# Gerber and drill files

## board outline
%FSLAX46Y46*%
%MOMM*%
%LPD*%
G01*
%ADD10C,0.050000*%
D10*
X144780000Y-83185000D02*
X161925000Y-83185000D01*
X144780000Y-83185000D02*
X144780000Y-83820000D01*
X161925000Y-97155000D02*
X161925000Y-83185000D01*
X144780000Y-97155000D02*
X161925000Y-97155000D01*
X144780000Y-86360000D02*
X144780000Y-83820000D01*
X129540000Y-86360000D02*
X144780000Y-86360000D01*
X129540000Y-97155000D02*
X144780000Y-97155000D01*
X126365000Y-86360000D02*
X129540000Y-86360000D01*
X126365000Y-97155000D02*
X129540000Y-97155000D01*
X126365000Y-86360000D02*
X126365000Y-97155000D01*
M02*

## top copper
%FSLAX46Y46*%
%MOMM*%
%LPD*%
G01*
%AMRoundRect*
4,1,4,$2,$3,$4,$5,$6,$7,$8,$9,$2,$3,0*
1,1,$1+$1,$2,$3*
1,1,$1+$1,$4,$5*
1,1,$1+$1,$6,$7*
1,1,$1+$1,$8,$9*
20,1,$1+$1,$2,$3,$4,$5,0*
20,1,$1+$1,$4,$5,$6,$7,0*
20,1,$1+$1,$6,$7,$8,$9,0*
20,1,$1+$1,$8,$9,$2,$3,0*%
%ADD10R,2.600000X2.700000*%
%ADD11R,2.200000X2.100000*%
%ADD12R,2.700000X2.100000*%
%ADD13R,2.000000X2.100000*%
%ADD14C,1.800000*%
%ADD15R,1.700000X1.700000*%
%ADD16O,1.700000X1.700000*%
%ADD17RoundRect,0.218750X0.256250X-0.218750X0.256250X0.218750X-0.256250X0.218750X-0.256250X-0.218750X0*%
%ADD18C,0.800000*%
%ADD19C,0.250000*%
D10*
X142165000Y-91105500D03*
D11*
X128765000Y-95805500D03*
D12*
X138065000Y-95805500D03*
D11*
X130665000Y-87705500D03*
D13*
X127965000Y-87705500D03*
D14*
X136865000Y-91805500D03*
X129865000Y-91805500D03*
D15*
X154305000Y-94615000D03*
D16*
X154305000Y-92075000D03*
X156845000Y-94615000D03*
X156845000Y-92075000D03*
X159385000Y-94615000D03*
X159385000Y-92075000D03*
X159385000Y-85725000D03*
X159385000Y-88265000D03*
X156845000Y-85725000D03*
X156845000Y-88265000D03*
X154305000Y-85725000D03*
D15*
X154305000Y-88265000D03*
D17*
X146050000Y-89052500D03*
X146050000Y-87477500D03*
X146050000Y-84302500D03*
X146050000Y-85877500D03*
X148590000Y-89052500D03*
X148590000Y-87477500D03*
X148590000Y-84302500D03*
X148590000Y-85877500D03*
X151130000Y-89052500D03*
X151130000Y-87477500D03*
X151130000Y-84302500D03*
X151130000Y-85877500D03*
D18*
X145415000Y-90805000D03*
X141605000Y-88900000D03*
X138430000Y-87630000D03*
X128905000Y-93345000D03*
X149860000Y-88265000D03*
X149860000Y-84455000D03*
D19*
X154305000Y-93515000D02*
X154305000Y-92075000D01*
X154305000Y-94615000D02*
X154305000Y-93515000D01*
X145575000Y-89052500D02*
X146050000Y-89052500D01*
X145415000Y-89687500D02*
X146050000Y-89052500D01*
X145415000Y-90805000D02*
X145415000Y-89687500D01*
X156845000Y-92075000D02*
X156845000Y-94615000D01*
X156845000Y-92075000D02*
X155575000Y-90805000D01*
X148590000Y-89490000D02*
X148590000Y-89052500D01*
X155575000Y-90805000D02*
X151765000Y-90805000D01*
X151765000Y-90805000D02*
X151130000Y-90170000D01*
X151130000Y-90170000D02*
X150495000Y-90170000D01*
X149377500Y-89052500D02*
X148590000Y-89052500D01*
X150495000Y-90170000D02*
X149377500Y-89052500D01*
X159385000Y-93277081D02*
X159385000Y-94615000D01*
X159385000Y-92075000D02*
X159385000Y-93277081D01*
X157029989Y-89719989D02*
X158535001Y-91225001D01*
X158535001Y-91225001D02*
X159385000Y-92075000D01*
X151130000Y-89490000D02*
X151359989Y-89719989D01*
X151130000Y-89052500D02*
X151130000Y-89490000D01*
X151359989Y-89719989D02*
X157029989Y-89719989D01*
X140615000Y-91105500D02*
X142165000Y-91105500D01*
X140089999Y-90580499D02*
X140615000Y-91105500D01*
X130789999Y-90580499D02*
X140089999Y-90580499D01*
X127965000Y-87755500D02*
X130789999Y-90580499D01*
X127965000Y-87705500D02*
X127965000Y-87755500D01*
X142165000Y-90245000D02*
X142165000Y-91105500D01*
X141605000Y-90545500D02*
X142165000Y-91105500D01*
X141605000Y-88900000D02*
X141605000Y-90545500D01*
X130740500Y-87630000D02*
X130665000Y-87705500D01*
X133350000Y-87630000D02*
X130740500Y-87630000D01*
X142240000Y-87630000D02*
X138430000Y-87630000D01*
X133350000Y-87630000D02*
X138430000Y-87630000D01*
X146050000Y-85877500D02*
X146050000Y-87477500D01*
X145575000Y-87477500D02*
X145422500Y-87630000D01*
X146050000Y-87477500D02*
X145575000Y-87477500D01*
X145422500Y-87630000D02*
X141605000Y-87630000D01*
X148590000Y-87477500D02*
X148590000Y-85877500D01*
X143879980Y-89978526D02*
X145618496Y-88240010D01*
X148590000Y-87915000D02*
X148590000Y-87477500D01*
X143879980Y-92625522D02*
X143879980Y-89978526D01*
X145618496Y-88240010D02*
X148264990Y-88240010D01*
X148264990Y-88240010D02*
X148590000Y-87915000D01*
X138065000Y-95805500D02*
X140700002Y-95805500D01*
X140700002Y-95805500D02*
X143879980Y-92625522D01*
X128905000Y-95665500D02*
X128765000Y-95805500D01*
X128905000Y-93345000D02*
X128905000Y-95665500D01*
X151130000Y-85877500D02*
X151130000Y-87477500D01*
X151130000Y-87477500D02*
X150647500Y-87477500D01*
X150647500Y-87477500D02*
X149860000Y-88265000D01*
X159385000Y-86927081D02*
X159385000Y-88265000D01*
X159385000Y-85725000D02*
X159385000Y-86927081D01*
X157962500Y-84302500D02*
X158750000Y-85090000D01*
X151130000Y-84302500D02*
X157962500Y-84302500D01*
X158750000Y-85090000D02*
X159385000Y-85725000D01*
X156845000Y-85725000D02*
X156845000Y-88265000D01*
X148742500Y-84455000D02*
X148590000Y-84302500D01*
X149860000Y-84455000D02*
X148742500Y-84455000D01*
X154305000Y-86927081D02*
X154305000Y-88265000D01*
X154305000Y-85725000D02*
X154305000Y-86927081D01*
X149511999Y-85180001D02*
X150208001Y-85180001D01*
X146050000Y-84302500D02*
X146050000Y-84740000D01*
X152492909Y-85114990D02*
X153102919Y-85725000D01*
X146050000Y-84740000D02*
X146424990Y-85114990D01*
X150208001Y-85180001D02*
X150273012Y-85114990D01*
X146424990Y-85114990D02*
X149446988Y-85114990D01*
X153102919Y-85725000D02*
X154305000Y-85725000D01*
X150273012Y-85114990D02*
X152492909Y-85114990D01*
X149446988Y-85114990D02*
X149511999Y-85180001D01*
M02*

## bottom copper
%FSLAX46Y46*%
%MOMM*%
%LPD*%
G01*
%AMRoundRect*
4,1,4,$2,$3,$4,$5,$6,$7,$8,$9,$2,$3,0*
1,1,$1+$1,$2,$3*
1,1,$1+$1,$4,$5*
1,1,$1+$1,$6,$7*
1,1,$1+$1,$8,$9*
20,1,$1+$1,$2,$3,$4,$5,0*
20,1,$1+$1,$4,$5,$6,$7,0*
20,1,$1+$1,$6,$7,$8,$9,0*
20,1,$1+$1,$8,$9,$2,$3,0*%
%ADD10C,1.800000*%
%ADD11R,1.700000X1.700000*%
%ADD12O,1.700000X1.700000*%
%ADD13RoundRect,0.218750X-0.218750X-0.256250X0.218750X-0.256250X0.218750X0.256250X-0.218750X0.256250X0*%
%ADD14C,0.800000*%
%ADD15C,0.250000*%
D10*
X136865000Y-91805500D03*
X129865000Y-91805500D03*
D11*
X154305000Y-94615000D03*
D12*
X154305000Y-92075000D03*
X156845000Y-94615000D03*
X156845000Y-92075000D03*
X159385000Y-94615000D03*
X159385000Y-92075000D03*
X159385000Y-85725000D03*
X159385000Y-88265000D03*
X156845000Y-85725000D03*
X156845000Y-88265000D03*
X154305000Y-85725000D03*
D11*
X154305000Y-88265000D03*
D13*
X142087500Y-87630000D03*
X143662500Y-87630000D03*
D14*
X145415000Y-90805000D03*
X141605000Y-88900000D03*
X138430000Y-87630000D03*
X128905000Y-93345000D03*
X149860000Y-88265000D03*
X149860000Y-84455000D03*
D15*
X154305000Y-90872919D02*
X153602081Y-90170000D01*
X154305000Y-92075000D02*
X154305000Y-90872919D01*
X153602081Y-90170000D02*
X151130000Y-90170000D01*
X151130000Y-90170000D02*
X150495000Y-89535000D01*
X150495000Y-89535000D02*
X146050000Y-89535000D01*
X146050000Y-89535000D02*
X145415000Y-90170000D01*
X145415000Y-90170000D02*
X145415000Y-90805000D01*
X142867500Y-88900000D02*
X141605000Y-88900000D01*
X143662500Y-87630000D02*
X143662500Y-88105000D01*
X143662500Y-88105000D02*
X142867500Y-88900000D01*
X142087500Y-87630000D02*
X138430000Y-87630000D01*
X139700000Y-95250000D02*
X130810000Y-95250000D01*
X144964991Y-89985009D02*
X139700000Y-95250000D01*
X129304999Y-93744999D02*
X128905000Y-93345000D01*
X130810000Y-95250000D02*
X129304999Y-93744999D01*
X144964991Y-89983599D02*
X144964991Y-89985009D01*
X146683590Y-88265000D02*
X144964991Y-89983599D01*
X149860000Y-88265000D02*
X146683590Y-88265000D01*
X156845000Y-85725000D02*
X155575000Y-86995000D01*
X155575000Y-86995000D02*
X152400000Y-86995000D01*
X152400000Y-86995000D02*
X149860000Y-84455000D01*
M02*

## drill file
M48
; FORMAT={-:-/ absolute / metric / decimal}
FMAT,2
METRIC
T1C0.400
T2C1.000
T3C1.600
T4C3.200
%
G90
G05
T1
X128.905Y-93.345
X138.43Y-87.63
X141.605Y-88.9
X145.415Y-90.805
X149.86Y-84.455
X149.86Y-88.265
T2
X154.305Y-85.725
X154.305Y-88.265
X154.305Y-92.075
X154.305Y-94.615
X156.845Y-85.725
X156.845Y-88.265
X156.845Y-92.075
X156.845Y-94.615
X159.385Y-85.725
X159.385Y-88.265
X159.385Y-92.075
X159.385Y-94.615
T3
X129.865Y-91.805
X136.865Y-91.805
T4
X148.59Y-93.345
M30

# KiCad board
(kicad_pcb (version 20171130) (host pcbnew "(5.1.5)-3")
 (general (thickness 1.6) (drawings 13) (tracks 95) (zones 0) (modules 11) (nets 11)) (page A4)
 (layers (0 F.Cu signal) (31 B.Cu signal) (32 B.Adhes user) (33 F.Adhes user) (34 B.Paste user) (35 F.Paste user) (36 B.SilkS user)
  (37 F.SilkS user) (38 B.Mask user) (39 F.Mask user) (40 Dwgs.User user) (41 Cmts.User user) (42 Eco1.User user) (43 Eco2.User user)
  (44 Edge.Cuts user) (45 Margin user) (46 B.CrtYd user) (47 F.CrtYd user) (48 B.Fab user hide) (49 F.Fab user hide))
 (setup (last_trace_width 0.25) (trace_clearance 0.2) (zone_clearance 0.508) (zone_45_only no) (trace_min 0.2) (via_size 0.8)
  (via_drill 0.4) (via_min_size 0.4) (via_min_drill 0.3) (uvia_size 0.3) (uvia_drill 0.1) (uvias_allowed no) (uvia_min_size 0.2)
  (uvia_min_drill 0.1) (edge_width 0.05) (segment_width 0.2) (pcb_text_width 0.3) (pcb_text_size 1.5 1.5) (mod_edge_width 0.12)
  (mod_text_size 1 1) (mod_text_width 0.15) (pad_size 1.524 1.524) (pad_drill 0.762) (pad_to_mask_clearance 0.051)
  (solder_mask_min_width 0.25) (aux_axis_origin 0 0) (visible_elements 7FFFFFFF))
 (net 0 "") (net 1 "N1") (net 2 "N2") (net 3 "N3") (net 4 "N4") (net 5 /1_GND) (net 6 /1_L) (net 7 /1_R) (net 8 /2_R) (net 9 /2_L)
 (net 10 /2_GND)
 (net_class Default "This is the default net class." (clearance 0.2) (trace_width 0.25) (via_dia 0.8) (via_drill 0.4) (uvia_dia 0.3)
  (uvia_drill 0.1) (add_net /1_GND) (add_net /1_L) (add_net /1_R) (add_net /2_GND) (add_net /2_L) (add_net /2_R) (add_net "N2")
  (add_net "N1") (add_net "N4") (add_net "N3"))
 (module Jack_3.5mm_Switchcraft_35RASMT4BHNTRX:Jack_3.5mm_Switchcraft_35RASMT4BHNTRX (layer F.Cu) (at 126.365 94.8055)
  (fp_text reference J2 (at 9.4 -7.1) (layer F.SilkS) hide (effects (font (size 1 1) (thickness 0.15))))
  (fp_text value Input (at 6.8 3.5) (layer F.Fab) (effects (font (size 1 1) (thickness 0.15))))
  (pad RN smd rect (at 15.8 -3.7) (size 2.6 2.7) (layers F.Cu F.Paste F.Mask) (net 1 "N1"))
  (pad R smd rect (at 2.4 1) (size 2.2 2.1) (layers F.Cu F.Paste F.Mask) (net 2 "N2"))
  (pad T smd rect (at 11.7 1) (size 2.7 2.1) (layers F.Cu F.Paste F.Mask) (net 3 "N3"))
  (pad S smd rect (at 4.3 -7.1) (size 2.2 2.1) (layers F.Cu F.Paste F.Mask) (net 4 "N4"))
  (pad TN smd rect (at 1.6 -7.1) (size 2 2.1) (layers F.Cu F.Paste F.Mask) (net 1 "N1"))
  (pad "" np_thru_hole circle (at 10.5 -3) (size 1.8 1.8) (drill 1.6) (layers *.Cu *.Mask))
  (pad "" np_thru_hole circle (at 3.5 -3) (size 1.8 1.8) (drill 1.6) (layers *.Cu *.Mask)))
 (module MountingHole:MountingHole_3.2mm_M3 (layer F.Cu) (at 148.59 93.345)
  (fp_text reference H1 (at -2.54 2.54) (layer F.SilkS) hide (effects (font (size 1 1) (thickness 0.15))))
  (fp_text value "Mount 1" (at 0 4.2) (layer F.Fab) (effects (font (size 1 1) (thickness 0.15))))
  (pad 1 np_thru_hole circle (at 0 0) (size 3.2 3.2) (drill 3.2) (layers *.Cu *.Mask)))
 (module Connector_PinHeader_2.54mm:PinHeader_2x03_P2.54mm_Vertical (layer F.Cu) (at 154.305 94.615 90)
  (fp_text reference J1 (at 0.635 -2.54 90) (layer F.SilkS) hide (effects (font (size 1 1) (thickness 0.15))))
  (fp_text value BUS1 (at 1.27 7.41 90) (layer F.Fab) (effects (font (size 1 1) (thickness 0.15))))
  (pad 1 thru_hole rect (at 0 0 90) (size 1.7 1.7) (drill 1) (layers *.Cu *.Mask) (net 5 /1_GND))
  (pad 2 thru_hole oval (at 2.54 0 90) (size 1.7 1.7) (drill 1) (layers *.Cu *.Mask) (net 5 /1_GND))
  (pad 3 thru_hole oval (at 0 2.54 90) (size 1.7 1.7) (drill 1) (layers *.Cu *.Mask) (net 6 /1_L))
  (pad 4 thru_hole oval (at 2.54 2.54 90) (size 1.7 1.7) (drill 1) (layers *.Cu *.Mask) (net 6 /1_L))
  (pad 5 thru_hole oval (at 0 5.08 90) (size 1.7 1.7) (drill 1) (layers *.Cu *.Mask) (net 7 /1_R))
  (pad 6 thru_hole oval (at 2.54 5.08 90) (size 1.7 1.7) (drill 1) (layers *.Cu *.Mask) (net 7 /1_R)))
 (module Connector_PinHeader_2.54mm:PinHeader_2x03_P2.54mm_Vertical (layer F.Cu) (at 154.305 88.265 90)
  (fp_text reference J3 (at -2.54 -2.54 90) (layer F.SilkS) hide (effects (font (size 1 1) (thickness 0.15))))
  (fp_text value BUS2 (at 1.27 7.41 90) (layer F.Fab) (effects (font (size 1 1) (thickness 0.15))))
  (pad 6 thru_hole oval (at 2.54 5.08 90) (size 1.7 1.7) (drill 1) (layers *.Cu *.Mask) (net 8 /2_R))
  (pad 5 thru_hole oval (at 0 5.08 90) (size 1.7 1.7) (drill 1) (layers *.Cu *.Mask) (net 8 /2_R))
  (pad 4 thru_hole oval (at 2.54 2.54 90) (size 1.7 1.7) (drill 1) (layers *.Cu *.Mask) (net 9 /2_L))
  (pad 3 thru_hole oval (at 0 2.54 90) (size 1.7 1.7) (drill 1) (layers *.Cu *.Mask) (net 9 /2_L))
  (pad 2 thru_hole oval (at 2.54 0 90) (size 1.7 1.7) (drill 1) (layers *.Cu *.Mask) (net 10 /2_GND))
  (pad 1 thru_hole rect (at 0 0 90) (size 1.7 1.7) (drill 1) (layers *.Cu *.Mask) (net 10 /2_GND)))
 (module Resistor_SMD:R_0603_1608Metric (layer F.Cu) (at 146.05 88.265 90)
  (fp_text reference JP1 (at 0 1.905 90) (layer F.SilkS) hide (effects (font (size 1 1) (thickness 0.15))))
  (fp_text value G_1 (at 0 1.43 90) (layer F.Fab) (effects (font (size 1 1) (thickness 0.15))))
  (pad 1 smd roundrect (at -0.7875 0 90) (size 0.875 0.95) (layers F.Cu F.Paste F.Mask) (roundrect_rratio 0.25) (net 5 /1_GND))
  (pad 2 smd roundrect (at 0.7875 0 90) (size 0.875 0.95) (layers F.Cu F.Paste F.Mask) (roundrect_rratio 0.25) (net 4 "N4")))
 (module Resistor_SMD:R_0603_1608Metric (layer F.Cu) (at 146.05 85.09 90)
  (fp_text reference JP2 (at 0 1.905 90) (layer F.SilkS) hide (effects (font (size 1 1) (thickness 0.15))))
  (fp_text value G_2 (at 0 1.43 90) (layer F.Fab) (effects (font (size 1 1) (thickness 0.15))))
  (pad 2 smd roundrect (at 0.7875 0 90) (size 0.875 0.95) (layers F.Cu F.Paste F.Mask) (roundrect_rratio 0.25) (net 10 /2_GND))
  (pad 1 smd roundrect (at -0.7875 0 90) (size 0.875 0.95) (layers F.Cu F.Paste F.Mask) (roundrect_rratio 0.25) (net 4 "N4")))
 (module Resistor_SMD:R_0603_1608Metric (layer F.Cu) (at 148.59 88.265 90)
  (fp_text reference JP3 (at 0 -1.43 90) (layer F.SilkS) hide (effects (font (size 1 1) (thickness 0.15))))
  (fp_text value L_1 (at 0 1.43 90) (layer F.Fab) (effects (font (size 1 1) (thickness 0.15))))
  (pad 1 smd roundrect (at -0.7875 0 90) (size 0.875 0.95) (layers F.Cu F.Paste F.Mask) (roundrect_rratio 0.25) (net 6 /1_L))
  (pad 2 smd roundrect (at 0.7875 0 90) (size 0.875 0.95) (layers F.Cu F.Paste F.Mask) (roundrect_rratio 0.25) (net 3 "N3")))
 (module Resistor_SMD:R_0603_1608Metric (layer F.Cu) (at 148.59 85.09 90)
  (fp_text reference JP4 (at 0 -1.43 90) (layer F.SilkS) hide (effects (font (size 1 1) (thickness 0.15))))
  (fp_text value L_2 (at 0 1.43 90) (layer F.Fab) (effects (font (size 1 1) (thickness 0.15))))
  (pad 2 smd roundrect (at 0.7875 0 90) (size 0.875 0.95) (layers F.Cu F.Paste F.Mask) (roundrect_rratio 0.25) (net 9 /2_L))
  (pad 1 smd roundrect (at -0.7875 0 90) (size 0.875 0.95) (layers F.Cu F.Paste F.Mask) (roundrect_rratio 0.25) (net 3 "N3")))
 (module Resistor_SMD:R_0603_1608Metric (layer F.Cu) (at 151.13 88.265 90)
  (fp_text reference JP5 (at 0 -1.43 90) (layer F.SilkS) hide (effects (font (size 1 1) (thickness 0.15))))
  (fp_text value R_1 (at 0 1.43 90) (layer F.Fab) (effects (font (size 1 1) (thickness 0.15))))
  (pad 1 smd roundrect (at -0.7875 0 90) (size 0.875 0.95) (layers F.Cu F.Paste F.Mask) (roundrect_rratio 0.25) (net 7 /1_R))
  (pad 2 smd roundrect (at 0.7875 0 90) (size 0.875 0.95) (layers F.Cu F.Paste F.Mask) (roundrect_rratio 0.25) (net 2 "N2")))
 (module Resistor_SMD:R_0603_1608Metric (layer F.Cu) (at 151.13 85.09 90)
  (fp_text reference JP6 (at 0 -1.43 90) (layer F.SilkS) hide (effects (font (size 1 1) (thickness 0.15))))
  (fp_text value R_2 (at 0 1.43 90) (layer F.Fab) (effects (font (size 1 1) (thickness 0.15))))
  (pad 2 smd roundrect (at 0.7875 0 90) (size 0.875 0.95) (layers F.Cu F.Paste F.Mask) (roundrect_rratio 0.25) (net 8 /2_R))
  (pad 1 smd roundrect (at -0.7875 0 90) (size 0.875 0.95) (layers F.Cu F.Paste F.Mask) (roundrect_rratio 0.25) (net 2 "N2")))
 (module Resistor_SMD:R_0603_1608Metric (layer B.Cu) (at 142.875 87.63)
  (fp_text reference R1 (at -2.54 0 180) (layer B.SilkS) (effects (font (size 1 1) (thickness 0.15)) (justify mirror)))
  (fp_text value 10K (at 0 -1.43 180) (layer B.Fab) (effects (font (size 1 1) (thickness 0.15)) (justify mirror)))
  (pad 1 smd roundrect (at -0.7875 0) (size 0.875 0.95) (layers B.Cu B.Paste B.Mask) (roundrect_rratio 0.25) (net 4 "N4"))
  (pad 2 smd roundrect (at 0.7875 0) (size 0.875 0.95) (layers B.Cu B.Paste B.Mask) (roundrect_rratio 0.25) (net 1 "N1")))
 (gr_line (start 144.78 83.185) (end 161.925 83.185) (layer Edge.Cuts) (width 0.05))
 (gr_line (start 144.78 83.185) (end 144.78 83.82) (layer Edge.Cuts) (width 0.05))
 (gr_line (start 161.925 97.155) (end 161.925 83.185) (layer Edge.Cuts) (width 0.05))
 (gr_line (start 144.78 97.155) (end 161.925 97.155) (layer Edge.Cuts) (width 0.05))
 (gr_line (start 144.78 86.36) (end 144.78 83.82) (layer Edge.Cuts) (width 0.05))
 (gr_line (start 129.54 86.36) (end 144.78 86.36) (layer Edge.Cuts) (width 0.05))
 (gr_line (start 129.54 97.155) (end 144.78 97.155) (layer Edge.Cuts) (width 0.05))
 (gr_line (start 126.365 86.36) (end 129.54 86.36) (layer Edge.Cuts) (width 0.05))
 (gr_line (start 126.365 97.155) (end 129.54 97.155) (layer Edge.Cuts) (width 0.05))
 (gr_line (start 126.365 86.36) (end 126.365 97.155) (layer Edge.Cuts) (width 0.05))
 (segment (start 154.305 93.515) (end 154.305 92.075) (width 0.25) (layer F.Cu) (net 5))
 (segment (start 154.305 94.615) (end 154.305 93.515) (width 0.25) (layer F.Cu) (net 5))
 (segment (start 145.575 89.0525) (end 146.05 89.0525) (width 0.25) (layer F.Cu) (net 5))
 (segment (start 154.305 90.872919) (end 153.602081 90.17) (width 0.25) (layer B.Cu) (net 5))
 (segment (start 154.305 92.075) (end 154.305 90.872919) (width 0.25) (layer B.Cu) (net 5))
 (segment (start 153.602081 90.17) (end 151.13 90.17) (width 0.25) (layer B.Cu) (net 5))
 (segment (start 151.13 90.17) (end 150.495 89.535) (width 0.25) (layer B.Cu) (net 5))
 (segment (start 150.495 89.535) (end 146.05 89.535) (width 0.25) (layer B.Cu) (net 5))
 (via (at 145.415 90.805) (size 0.8) (drill 0.4) (layers F.Cu B.Cu) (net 5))
 (segment (start 146.05 89.535) (end 145.415 90.17) (width 0.25) (layer B.Cu) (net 5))
 (segment (start 145.415 90.17) (end 145.415 90.805) (width 0.25) (layer B.Cu) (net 5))
 (segment (start 145.415 89.6875) (end 146.05 89.0525) (width 0.25) (layer F.Cu) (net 5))
 (segment (start 145.415 90.805) (end 145.415 89.6875) (width 0.25) (layer F.Cu) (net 5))
 (segment (start 156.845 92.075) (end 156.845 94.615) (width 0.25) (layer F.Cu) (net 6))
 (segment (start 156.845 92.075) (end 155.575 90.805) (width 0.25) (layer F.Cu) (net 6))
 (segment (start 148.59 89.49) (end 148.59 89.0525) (width 0.25) (layer F.Cu) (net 6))
 (segment (start 155.575 90.805) (end 151.765 90.805) (width 0.25) (layer F.Cu) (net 6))
 (segment (start 151.765 90.805) (end 151.13 90.17) (width 0.25) (layer F.Cu) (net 6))
 (segment (start 151.13 90.17) (end 150.495 90.17) (width 0.25) (layer F.Cu) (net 6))
 (segment (start 149.3775 89.0525) (end 148.59 89.0525) (width 0.25) (layer F.Cu) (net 6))
 (segment (start 150.495 90.17) (end 149.3775 89.0525) (width 0.25) (layer F.Cu) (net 6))
 (segment (start 159.385 93.277081) (end 159.385 94.615) (width 0.25) (layer F.Cu) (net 7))
 (segment (start 159.385 92.075) (end 159.385 93.277081) (width 0.25) (layer F.Cu) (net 7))
 (segment (start 157.029989 89.719989) (end 158.535001 91.225001) (width 0.25) (layer F.Cu) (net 7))
 (segment (start 158.535001 91.225001) (end 159.385 92.075) (width 0.25) (layer F.Cu) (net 7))
 (segment (start 151.13 89.49) (end 151.359989 89.719989) (width 0.25) (layer F.Cu) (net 7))
 (segment (start 151.13 89.0525) (end 151.13 89.49) (width 0.25) (layer F.Cu) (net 7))
 (segment (start 151.359989 89.719989) (end 157.029989 89.719989) (width 0.25) (layer F.Cu) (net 7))
 (segment (start 140.615 91.1055) (end 142.165 91.1055) (width 0.25) (layer F.Cu) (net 1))
 (segment (start 140.089999 90.580499) (end 140.615 91.1055) (width 0.25) (layer F.Cu) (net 1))
 (segment (start 130.789999 90.580499) (end 140.089999 90.580499) (width 0.25) (layer F.Cu) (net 1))
 (segment (start 127.965 87.7555) (end 130.789999 90.580499) (width 0.25) (layer F.Cu) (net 1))
 (segment (start 127.965 87.7055) (end 127.965 87.7555) (width 0.25) (layer F.Cu) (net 1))
 (segment (start 142.165 90.245) (end 142.165 91.1055) (width 0.25) (layer F.Cu) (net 1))
 (via (at 141.605 88.9) (size 0.8) (drill 0.4) (layers F.Cu B.Cu) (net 1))
 (segment (start 142.8675 88.9) (end 141.605 88.9) (width 0.25) (layer B.Cu) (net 1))
 (segment (start 143.6625 87.63) (end 143.6625 88.105) (width 0.25) (layer B.Cu) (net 1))
 (segment (start 143.6625 88.105) (end 142.8675 88.9) (width 0.25) (layer B.Cu) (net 1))
 (segment (start 141.605 90.5455) (end 142.165 91.1055) (width 0.25) (layer F.Cu) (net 1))
 (segment (start 141.605 88.9) (end 141.605 90.5455) (width 0.25) (layer F.Cu) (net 1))
 (segment (start 130.7405 87.63) (end 130.665 87.7055) (width 0.25) (layer F.Cu) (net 4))
 (segment (start 133.35 87.63) (end 130.7405 87.63) (width 0.25) (layer F.Cu) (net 4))
 (via (at 138.43 87.63) (size 0.8) (drill 0.4) (layers F.Cu B.Cu) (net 4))
 (segment (start 142.24 87.63) (end 138.43 87.63) (width 0.25) (layer F.Cu) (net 4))
 (segment (start 142.0875 87.63) (end 138.43 87.63) (width 0.25) (layer B.Cu) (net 4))
 (segment (start 133.35 87.63) (end 138.43 87.63) (width 0.25) (layer F.Cu) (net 4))
 (segment (start 146.05 85.8775) (end 146.05 87.4775) (width 0.25) (layer F.Cu) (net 4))
 (segment (start 145.575 87.4775) (end 145.4225 87.63) (width 0.25) (layer F.Cu) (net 4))
 (segment (start 146.05 87.4775) (end 145.575 87.4775) (width 0.25) (layer F.Cu) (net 4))
 (segment (start 145.4225 87.63) (end 141.605 87.63) (width 0.25) (layer F.Cu) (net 4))
 (segment (start 148.59 87.4775) (end 148.59 85.8775) (width 0.25) (layer F.Cu) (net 3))
 (segment (start 143.87998 89.978526) (end 145.618496 88.24001) (width 0.25) (layer F.Cu) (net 3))
 (segment (start 148.59 87.915) (end 148.59 87.4775) (width 0.25) (layer F.Cu) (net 3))
 (segment (start 143.87998 92.625522) (end 143.87998 89.978526) (width 0.25) (layer F.Cu) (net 3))
 (segment (start 145.618496 88.24001) (end 148.26499 88.24001) (width 0.25) (layer F.Cu) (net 3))
 (segment (start 148.26499 88.24001) (end 148.59 87.915) (width 0.25) (layer F.Cu) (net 3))
 (segment (start 138.065 95.8055) (end 140.700002 95.8055) (width 0.25) (layer F.Cu) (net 3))
 (segment (start 140.700002 95.8055) (end 143.87998 92.625522) (width 0.25) (layer F.Cu) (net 3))
 (via (at 128.905 93.345) (size 0.8) (drill 0.4) (layers F.Cu B.Cu) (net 2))
 (segment (start 128.905 95.6655) (end 128.765 95.8055) (width 0.25) (layer F.Cu) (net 2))
 (segment (start 128.905 93.345) (end 128.905 95.6655) (width 0.25) (layer F.Cu) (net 2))
 (segment (start 151.13 85.8775) (end 151.13 87.4775) (width 0.25) (layer F.Cu) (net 2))
 (via (at 149.86 88.265) (size 0.8) (drill 0.4) (layers F.Cu B.Cu) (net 2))
 (segment (start 151.13 87.4775) (end 150.6475 87.4775) (width 0.25) (layer F.Cu) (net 2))
 (segment (start 150.6475 87.4775) (end 149.86 88.265) (width 0.25) (layer F.Cu) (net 2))
 (segment (start 139.7 95.25) (end 130.81 95.25) (width 0.25) (layer B.Cu) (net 2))
 (segment (start 144.964991 89.985009) (end 139.7 95.25) (width 0.25) (layer B.Cu) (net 2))
 (segment (start 129.304999 93.744999) (end 128.905 93.345) (width 0.25) (layer B.Cu) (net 2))
 (segment (start 130.81 95.25) (end 129.304999 93.744999) (width 0.25) (layer B.Cu) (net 2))
 (segment (start 144.964991 89.983599) (end 144.964991 89.985009) (width 0.25) (layer B.Cu) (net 2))
 (segment (start 146.68359 88.265) (end 144.964991 89.983599) (width 0.25) (layer B.Cu) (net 2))
 (segment (start 149.86 88.265) (end 146.68359 88.265) (width 0.25) (layer B.Cu) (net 2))
 (segment (start 159.385 86.927081) (end 159.385 88.265) (width 0.25) (layer F.Cu) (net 8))
 (segment (start 159.385 85.725) (end 159.385 86.927081) (width 0.25) (layer F.Cu) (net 8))
 (segment (start 157.9625 84.3025) (end 158.75 85.09) (width 0.25) (layer F.Cu) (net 8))
 (segment (start 151.13 84.3025) (end 157.9625 84.3025) (width 0.25) (layer F.Cu) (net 8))
 (segment (start 158.75 85.09) (end 159.385 85.725) (width 0.25) (layer F.Cu) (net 8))
 (segment (start 156.845 85.725) (end 156.845 88.265) (width 0.25) (layer F.Cu) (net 9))
 (segment (start 156.845 85.725) (end 155.575 86.995) (width 0.25) (layer B.Cu) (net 9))
 (segment (start 155.575 86.995) (end 152.4 86.995) (width 0.25) (layer B.Cu) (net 9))
 (via (at 149.86 84.455) (size 0.8) (drill 0.4) (layers F.Cu B.Cu) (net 9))
 (segment (start 152.4 86.995) (end 149.86 84.455) (width 0.25) (layer B.Cu) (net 9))
 (segment (start 148.7425 84.455) (end 148.59 84.3025) (width 0.25) (layer F.Cu) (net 9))
 (segment (start 149.86 84.455) (end 148.7425 84.455) (width 0.25) (layer F.Cu) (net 9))
 (segment (start 154.305 86.927081) (end 154.305 88.265) (width 0.25) (layer F.Cu) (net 10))
 (segment (start 154.305 85.725) (end 154.305 86.927081) (width 0.25) (layer F.Cu) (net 10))
 (segment (start 149.511999 85.180001) (end 150.208001 85.180001) (width 0.25) (layer F.Cu) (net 10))
 (segment (start 146.05 84.3025) (end 146.05 84.74) (width 0.25) (layer F.Cu) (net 10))
 (segment (start 152.492909 85.11499) (end 153.102919 85.725) (width 0.25) (layer F.Cu) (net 10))
 (segment (start 146.05 84.74) (end 146.42499 85.11499) (width 0.25) (layer F.Cu) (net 10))
 (segment (start 150.208001 85.180001) (end 150.273012 85.11499) (width 0.25) (layer F.Cu) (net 10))
 (segment (start 146.42499 85.11499) (end 149.446988 85.11499) (width 0.25) (layer F.Cu) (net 10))
 (segment (start 153.102919 85.725) (end 154.305 85.725) (width 0.25) (layer F.Cu) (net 10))
 (segment (start 150.273012 85.11499) (end 152.492909 85.11499) (width 0.25) (layer F.Cu) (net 10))
 (segment (start 149.446988 85.11499) (end 149.511999 85.180001) (width 0.25) (layer F.Cu) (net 10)))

